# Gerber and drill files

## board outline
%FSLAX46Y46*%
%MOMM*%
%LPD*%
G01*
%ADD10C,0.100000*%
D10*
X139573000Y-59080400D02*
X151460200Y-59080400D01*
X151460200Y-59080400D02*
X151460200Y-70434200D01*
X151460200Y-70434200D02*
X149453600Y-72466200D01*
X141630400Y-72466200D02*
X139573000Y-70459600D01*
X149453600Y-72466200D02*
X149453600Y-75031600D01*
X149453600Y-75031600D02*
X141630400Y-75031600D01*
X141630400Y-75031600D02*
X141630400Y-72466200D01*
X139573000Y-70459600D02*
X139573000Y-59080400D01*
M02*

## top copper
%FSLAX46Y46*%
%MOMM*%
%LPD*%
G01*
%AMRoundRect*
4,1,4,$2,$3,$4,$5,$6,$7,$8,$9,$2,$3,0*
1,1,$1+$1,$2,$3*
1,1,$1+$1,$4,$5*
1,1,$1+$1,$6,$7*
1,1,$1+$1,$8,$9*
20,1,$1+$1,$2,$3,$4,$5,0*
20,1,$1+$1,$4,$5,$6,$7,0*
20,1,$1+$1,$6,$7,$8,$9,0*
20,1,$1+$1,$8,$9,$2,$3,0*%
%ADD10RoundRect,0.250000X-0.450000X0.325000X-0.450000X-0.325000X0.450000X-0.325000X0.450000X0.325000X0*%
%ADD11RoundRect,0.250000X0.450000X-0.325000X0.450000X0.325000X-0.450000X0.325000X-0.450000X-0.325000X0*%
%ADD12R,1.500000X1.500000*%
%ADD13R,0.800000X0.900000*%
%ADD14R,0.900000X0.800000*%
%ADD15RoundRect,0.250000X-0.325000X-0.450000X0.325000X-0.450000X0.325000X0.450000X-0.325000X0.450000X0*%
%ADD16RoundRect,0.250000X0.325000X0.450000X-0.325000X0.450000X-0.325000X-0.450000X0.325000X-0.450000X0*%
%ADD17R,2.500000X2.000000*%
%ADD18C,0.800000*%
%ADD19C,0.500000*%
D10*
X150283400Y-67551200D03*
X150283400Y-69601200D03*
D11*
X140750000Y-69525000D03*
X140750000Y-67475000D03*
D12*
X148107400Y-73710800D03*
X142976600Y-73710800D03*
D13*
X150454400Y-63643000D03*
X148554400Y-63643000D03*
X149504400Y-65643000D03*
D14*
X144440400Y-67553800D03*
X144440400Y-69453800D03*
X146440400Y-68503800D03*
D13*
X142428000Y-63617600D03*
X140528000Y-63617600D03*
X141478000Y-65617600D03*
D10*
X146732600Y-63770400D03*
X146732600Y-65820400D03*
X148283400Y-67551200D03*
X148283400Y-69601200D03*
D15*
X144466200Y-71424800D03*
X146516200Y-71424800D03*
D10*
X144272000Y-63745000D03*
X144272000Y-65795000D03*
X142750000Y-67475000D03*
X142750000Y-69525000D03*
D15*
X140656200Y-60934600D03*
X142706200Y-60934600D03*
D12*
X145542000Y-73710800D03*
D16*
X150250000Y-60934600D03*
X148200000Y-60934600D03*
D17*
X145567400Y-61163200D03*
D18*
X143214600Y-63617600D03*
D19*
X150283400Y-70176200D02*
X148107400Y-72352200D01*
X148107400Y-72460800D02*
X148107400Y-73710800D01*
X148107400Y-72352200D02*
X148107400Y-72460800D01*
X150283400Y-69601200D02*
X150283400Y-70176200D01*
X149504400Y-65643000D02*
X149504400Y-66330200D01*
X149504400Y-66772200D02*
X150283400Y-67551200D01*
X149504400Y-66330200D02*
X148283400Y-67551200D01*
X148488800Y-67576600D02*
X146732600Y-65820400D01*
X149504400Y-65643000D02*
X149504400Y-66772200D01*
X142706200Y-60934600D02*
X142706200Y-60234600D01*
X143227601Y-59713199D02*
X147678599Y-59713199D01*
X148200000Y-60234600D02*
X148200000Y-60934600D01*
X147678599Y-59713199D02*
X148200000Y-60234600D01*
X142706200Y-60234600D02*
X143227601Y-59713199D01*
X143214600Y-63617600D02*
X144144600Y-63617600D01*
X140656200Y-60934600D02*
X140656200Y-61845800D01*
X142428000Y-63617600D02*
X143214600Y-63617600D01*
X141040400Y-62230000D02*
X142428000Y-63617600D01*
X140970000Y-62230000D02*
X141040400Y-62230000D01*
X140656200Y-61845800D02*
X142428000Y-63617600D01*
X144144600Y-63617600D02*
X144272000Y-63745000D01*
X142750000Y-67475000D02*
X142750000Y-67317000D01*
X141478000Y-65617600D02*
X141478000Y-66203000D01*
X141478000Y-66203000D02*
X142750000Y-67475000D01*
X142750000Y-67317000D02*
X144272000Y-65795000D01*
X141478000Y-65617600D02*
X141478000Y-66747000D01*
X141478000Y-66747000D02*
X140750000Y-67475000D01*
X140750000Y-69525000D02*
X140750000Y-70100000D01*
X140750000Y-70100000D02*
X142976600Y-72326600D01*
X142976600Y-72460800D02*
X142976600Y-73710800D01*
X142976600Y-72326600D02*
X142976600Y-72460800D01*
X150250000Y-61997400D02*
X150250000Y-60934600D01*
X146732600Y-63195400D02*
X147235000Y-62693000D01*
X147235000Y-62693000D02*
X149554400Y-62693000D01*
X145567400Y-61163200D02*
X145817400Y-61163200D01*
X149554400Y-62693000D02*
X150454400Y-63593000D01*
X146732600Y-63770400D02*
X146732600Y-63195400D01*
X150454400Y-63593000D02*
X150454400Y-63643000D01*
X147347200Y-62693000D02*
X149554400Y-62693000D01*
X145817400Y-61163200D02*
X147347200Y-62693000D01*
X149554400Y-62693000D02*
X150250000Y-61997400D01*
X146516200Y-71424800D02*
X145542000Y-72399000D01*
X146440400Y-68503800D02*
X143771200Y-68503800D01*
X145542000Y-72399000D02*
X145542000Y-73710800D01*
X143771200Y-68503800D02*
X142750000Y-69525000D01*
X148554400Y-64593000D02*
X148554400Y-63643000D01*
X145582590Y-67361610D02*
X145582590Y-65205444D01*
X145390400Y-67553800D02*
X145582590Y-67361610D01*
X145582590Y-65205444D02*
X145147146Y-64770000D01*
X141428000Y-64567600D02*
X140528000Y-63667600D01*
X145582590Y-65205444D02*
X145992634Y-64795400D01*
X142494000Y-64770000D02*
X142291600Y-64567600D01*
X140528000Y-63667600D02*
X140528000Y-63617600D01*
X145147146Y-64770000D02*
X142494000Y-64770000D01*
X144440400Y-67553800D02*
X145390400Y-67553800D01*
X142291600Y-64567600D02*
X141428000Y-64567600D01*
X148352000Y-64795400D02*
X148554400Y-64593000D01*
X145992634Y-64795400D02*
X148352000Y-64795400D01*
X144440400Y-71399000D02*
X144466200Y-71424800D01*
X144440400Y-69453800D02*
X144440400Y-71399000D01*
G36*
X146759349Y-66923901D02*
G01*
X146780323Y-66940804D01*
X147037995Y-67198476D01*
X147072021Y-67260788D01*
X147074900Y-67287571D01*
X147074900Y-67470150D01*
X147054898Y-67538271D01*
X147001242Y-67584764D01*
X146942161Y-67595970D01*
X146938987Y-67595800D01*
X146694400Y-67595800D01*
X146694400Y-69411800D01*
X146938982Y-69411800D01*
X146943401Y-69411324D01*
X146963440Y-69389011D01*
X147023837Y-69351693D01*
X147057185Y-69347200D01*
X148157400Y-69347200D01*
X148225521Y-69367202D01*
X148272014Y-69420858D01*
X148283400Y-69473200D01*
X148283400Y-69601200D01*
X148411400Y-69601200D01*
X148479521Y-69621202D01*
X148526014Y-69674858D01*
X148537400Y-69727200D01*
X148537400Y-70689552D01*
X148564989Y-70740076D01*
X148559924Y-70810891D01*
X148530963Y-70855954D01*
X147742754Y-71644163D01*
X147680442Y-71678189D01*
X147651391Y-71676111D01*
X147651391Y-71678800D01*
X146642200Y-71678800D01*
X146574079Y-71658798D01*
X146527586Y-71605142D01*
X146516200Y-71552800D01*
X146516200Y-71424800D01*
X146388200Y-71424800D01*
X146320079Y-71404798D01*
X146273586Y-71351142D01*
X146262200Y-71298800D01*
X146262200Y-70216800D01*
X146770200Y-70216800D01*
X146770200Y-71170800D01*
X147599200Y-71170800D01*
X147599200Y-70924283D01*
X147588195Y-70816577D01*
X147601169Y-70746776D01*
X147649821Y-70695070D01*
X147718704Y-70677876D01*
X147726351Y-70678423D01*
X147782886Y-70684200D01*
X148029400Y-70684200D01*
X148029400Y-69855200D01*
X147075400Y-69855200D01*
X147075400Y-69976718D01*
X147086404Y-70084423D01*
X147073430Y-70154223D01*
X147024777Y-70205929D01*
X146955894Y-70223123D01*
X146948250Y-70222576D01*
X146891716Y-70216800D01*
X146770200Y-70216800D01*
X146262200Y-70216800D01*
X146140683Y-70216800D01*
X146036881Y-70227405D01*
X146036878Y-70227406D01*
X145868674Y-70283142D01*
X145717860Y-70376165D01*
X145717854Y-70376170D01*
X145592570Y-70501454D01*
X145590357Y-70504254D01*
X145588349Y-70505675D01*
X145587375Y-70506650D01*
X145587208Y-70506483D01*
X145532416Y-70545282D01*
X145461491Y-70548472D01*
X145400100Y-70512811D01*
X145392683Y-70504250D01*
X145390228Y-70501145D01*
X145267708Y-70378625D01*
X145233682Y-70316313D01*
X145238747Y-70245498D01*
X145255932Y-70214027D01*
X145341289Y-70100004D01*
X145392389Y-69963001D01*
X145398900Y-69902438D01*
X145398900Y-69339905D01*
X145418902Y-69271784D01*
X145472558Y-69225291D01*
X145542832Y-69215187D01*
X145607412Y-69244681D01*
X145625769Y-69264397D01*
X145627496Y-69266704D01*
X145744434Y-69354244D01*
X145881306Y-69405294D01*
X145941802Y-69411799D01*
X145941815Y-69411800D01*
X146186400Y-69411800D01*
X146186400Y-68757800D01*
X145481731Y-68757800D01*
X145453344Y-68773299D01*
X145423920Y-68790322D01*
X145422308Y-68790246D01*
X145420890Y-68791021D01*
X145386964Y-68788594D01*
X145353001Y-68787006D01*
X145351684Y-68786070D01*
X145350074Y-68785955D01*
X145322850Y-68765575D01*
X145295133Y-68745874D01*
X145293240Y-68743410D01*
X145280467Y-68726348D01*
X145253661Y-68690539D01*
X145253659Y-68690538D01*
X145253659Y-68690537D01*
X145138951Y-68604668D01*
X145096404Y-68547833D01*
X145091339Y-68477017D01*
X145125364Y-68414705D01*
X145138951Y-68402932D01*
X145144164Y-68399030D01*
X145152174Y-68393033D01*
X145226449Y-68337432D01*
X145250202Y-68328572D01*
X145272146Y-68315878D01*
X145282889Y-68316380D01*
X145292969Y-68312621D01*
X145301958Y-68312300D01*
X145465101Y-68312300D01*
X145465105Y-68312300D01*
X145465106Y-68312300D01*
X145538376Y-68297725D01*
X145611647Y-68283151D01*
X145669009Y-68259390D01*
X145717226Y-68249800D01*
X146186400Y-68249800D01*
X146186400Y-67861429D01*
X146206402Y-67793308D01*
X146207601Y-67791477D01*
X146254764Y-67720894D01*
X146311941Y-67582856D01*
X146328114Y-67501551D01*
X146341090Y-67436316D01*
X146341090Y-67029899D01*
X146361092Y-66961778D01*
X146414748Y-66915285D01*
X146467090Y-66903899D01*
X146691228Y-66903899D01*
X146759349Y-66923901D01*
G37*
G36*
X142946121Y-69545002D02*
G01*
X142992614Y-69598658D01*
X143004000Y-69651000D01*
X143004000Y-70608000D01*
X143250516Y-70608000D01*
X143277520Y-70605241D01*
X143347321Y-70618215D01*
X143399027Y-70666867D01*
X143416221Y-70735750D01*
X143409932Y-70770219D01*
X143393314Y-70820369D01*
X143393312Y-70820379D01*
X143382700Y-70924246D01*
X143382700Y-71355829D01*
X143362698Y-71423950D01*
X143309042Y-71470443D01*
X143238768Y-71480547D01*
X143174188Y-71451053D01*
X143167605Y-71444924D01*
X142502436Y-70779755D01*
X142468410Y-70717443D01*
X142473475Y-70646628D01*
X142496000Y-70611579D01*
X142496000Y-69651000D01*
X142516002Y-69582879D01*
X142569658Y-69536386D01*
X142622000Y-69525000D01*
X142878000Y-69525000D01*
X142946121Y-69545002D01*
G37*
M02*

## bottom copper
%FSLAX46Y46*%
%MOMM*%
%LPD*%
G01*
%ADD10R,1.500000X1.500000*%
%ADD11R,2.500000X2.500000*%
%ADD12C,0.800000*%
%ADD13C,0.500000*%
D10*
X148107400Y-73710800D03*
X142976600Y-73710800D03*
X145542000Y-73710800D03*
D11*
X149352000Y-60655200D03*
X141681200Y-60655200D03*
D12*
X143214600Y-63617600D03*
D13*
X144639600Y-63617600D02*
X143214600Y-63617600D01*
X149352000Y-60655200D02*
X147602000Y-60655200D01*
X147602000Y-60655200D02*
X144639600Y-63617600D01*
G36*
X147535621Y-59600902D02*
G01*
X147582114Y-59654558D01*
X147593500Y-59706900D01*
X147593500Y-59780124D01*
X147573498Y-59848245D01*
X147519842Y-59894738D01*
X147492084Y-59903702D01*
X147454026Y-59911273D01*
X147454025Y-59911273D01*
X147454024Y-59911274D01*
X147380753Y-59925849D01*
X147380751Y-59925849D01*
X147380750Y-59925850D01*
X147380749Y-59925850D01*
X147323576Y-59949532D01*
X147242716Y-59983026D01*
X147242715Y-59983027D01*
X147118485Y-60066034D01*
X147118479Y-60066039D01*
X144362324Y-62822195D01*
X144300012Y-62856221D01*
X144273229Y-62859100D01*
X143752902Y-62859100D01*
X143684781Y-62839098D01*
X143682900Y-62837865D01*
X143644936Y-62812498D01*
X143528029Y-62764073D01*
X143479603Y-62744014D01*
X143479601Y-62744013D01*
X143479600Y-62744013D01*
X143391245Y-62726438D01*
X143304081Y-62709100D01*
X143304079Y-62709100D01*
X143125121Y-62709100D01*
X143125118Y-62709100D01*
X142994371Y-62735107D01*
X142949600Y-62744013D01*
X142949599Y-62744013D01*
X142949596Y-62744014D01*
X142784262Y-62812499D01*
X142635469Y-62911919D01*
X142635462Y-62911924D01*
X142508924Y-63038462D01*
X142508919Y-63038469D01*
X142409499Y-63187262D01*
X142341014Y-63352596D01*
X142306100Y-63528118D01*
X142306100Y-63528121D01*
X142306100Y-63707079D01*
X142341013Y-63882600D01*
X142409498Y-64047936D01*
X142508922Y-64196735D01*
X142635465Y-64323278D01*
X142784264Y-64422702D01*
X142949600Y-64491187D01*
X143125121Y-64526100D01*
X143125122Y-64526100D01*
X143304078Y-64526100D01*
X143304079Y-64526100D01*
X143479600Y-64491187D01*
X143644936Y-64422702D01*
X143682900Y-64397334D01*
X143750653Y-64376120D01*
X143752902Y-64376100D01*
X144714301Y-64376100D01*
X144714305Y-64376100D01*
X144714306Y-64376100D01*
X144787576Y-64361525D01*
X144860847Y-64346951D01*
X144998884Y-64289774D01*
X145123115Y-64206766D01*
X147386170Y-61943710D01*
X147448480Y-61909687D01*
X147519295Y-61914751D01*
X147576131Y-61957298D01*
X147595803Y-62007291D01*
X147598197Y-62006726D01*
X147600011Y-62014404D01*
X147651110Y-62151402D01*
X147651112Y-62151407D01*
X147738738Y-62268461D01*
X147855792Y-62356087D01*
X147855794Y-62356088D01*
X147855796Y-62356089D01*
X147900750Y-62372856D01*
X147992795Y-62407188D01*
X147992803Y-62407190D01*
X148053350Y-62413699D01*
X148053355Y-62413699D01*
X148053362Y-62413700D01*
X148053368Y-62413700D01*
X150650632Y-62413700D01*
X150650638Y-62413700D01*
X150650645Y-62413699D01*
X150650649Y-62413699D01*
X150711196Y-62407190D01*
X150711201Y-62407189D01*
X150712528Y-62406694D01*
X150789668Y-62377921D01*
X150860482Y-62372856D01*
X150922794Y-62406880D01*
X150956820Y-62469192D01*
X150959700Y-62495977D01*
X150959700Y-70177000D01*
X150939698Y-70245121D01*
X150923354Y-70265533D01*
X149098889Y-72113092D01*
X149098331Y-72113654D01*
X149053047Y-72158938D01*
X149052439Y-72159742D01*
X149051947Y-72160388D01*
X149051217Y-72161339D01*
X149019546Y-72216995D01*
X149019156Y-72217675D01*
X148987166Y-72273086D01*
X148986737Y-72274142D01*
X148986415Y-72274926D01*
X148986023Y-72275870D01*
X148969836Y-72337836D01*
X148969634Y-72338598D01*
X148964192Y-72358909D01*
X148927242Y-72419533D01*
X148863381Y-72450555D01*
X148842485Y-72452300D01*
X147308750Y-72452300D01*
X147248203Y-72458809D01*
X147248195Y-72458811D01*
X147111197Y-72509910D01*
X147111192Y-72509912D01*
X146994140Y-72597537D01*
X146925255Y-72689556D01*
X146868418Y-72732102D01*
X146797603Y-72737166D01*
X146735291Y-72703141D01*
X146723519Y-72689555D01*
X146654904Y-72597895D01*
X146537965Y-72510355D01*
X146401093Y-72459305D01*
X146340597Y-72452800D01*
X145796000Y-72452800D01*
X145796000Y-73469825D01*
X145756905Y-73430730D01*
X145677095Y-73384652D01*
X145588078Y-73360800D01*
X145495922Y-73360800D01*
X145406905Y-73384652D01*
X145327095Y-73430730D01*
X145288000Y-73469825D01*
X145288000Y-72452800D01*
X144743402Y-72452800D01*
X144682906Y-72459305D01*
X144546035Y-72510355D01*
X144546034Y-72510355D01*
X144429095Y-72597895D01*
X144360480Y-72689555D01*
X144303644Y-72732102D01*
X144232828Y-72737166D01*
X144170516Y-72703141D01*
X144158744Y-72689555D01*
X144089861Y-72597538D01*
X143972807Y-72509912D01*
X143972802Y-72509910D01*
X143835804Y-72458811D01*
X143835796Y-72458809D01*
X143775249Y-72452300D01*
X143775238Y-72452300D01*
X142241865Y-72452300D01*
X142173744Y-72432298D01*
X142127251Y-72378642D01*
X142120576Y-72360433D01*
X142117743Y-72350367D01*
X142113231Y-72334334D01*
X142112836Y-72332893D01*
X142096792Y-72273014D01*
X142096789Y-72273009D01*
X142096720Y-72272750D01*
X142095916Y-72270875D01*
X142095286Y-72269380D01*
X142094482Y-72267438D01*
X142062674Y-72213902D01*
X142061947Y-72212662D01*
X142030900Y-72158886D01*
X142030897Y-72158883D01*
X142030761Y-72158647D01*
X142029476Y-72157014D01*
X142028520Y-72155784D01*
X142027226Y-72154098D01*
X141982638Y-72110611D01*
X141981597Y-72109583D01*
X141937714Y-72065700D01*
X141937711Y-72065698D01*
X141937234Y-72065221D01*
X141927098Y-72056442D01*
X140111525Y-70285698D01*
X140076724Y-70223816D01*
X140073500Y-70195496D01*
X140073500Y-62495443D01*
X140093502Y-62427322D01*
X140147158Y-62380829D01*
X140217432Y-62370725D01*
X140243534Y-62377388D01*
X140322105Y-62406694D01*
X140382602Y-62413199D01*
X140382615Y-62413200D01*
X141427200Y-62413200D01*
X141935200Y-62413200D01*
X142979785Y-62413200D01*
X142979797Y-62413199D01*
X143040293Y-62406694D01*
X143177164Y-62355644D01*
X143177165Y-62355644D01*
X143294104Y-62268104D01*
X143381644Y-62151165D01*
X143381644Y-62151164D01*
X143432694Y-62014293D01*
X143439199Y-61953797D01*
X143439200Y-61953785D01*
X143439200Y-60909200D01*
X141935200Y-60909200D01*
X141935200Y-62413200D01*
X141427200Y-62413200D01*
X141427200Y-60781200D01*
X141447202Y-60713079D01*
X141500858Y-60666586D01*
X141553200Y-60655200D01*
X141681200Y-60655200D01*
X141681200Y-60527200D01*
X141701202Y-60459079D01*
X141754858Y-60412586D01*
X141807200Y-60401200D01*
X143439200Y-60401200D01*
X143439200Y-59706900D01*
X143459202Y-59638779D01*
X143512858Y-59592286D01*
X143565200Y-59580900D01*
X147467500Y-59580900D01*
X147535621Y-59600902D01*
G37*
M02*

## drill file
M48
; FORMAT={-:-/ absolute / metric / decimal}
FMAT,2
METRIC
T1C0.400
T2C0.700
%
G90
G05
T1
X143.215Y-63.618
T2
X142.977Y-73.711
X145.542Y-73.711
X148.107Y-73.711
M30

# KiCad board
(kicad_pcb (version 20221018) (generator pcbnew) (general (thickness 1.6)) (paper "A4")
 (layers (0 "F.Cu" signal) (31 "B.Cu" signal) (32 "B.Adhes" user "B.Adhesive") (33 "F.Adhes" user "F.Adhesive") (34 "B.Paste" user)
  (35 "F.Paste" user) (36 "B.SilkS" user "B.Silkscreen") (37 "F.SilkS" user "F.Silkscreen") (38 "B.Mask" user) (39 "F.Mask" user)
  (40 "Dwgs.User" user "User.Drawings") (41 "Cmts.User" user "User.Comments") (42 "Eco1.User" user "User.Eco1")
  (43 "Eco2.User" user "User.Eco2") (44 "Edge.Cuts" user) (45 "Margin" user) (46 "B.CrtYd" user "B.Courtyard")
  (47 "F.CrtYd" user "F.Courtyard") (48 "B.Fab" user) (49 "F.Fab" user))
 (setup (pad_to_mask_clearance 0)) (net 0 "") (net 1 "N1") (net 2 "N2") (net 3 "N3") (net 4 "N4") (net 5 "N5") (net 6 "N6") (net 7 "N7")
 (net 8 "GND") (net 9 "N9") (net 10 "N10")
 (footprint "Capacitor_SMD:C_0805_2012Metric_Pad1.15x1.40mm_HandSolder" (layer "F.Cu") (at 150.2834 68.5762 -90)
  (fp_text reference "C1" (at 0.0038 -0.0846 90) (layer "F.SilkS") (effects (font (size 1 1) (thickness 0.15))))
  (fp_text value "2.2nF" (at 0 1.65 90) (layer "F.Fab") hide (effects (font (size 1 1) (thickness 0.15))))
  (pad "1" smd roundrect (at -1.025 0 270) (size 1.15 1.4) (layers "F.Cu" "F.Paste" "F.Mask") (roundrect_rratio 0.217391) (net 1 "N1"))
  (pad "2" smd roundrect (at 1.025 0 270) (size 1.15 1.4) (layers "F.Cu" "F.Paste" "F.Mask") (roundrect_rratio 0.217391) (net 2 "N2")))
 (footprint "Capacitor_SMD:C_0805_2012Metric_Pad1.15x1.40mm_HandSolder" (layer "F.Cu") (at 140.75 68.5 90)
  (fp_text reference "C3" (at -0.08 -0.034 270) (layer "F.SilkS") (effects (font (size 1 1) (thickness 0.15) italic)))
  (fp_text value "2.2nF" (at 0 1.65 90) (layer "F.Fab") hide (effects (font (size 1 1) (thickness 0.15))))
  (pad "1" smd roundrect (at -1.025 0 90) (size 1.15 1.4) (layers "F.Cu" "F.Paste" "F.Mask") (roundrect_rratio 0.217391) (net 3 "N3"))
  (pad "2" smd roundrect (at 1.025 0 90) (size 1.15 1.4) (layers "F.Cu" "F.Paste" "F.Mask") (roundrect_rratio 0.217391) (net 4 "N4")))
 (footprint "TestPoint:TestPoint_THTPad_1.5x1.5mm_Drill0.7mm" (layer "F.Cu") (at 148.1074 73.7108)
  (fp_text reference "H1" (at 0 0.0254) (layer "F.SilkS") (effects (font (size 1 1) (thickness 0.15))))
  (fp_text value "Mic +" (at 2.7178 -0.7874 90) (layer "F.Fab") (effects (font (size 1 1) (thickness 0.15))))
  (pad "M-" thru_hole rect (at 0 0) (size 1.5 1.5) (drill 0.7) (layers "*.Cu" "*.Mask") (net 2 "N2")))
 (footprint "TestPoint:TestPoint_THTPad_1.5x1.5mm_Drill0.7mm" (layer "F.Cu") (at 142.9766 73.7108)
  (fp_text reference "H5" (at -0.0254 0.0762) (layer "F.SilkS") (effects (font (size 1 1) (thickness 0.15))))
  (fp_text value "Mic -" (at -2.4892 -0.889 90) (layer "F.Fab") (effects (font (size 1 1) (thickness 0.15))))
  (pad "M+" thru_hole rect (at 0 0) (size 1.5 1.5) (drill 0.7) (layers "*.Cu" "*.Mask") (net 3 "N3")))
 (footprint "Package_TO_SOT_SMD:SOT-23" (layer "F.Cu") (at 149.5044 64.643 -90)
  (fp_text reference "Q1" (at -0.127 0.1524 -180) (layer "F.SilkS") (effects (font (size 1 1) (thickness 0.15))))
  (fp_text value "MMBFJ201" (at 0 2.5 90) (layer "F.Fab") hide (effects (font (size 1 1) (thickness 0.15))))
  (pad "1" smd rect (at -1 -0.95 270) (size 0.9 0.8) (layers "F.Cu" "F.Paste" "F.Mask") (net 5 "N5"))
  (pad "2" smd rect (at -1 0.95 270) (size 0.9 0.8) (layers "F.Cu" "F.Paste" "F.Mask") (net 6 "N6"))
  (pad "3" smd rect (at 1 0 270) (size 0.9 0.8) (layers "F.Cu" "F.Paste" "F.Mask") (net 1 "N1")))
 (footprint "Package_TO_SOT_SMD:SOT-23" (layer "F.Cu") (at 145.4404 68.5038)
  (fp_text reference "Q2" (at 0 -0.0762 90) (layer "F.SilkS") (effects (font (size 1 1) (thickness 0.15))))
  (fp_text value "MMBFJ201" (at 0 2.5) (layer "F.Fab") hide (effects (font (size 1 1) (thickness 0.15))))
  (pad "1" smd rect (at -1 -0.95) (size 0.9 0.8) (layers "F.Cu" "F.Paste" "F.Mask") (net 6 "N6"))
  (pad "2" smd rect (at -1 0.95) (size 0.9 0.8) (layers "F.Cu" "F.Paste" "F.Mask") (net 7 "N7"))
  (pad "3" smd rect (at 1 0) (size 0.9 0.8) (layers "F.Cu" "F.Paste" "F.Mask") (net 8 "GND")))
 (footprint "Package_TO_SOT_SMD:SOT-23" (layer "F.Cu") (at 141.478 64.6176 -90)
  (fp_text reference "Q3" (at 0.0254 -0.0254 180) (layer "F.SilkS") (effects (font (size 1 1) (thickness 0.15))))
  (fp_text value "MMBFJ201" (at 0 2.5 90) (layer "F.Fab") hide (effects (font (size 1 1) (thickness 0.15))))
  (pad "1" smd rect (at -1 -0.95 270) (size 0.9 0.8) (layers "F.Cu" "F.Paste" "F.Mask") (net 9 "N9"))
  (pad "2" smd rect (at -1 0.95 270) (size 0.9 0.8) (layers "F.Cu" "F.Paste" "F.Mask") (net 6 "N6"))
  (pad "3" smd rect (at 1 0 270) (size 0.9 0.8) (layers "F.Cu" "F.Paste" "F.Mask") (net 4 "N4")))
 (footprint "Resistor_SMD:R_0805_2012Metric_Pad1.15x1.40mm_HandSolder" (layer "F.Cu") (at 146.7326 64.7954 -90)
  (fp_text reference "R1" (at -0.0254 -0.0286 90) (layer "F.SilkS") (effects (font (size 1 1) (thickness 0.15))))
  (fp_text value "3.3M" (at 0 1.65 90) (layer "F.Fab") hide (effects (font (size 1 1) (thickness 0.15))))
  (pad "1" smd roundrect (at -1.025 0 270) (size 1.15 1.4) (layers "F.Cu" "F.Paste" "F.Mask") (roundrect_rratio 0.217391) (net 5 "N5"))
  (pad "2" smd roundrect (at 1.025 0 270) (size 1.15 1.4) (layers "F.Cu" "F.Paste" "F.Mask") (roundrect_rratio 0.217391) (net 1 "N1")))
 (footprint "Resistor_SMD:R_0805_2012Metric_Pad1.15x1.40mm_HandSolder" (layer "F.Cu") (at 148.2834 68.5762 -90)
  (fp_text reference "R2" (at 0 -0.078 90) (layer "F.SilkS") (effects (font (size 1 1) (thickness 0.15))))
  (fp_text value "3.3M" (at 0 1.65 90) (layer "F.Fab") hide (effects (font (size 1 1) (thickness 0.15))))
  (pad "1" smd roundrect (at -1.025 0 270) (size 1.15 1.4) (layers "F.Cu" "F.Paste" "F.Mask") (roundrect_rratio 0.217391) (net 1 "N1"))
  (pad "2" smd roundrect (at 1.025 0 270) (size 1.15 1.4) (layers "F.Cu" "F.Paste" "F.Mask") (roundrect_rratio 0.217391) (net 8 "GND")))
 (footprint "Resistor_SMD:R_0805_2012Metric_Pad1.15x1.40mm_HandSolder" (layer "F.Cu") (at 145.4912 71.4248)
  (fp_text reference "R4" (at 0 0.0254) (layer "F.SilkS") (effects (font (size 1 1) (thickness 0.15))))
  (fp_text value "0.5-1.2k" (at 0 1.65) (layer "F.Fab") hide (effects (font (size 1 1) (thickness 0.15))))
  (pad "1" smd roundrect (at -1.025 0) (size 1.15 1.4) (layers "F.Cu" "F.Paste" "F.Mask") (roundrect_rratio 0.217391) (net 7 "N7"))
  (pad "2" smd roundrect (at 1.025 0) (size 1.15 1.4) (layers "F.Cu" "F.Paste" "F.Mask") (roundrect_rratio 0.217391) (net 8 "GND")))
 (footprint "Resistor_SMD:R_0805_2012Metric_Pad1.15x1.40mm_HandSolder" (layer "F.Cu") (at 144.272 64.77 -90)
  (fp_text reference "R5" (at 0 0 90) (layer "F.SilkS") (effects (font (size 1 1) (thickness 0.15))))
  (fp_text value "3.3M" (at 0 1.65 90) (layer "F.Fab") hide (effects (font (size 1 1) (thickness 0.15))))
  (pad "1" smd roundrect (at -1.025 0 270) (size 1.15 1.4) (layers "F.Cu" "F.Paste" "F.Mask") (roundrect_rratio 0.217391) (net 9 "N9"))
  (pad "2" smd roundrect (at 1.025 0 270) (size 1.15 1.4) (layers "F.Cu" "F.Paste" "F.Mask") (roundrect_rratio 0.217391) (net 4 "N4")))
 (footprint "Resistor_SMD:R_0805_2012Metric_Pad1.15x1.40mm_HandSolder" (layer "F.Cu") (at 142.75 68.5 -90)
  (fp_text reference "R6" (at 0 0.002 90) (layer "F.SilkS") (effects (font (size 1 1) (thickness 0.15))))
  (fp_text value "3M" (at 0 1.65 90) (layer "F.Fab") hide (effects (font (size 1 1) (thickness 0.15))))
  (pad "1" smd roundrect (at -1.025 0 270) (size 1.15 1.4) (layers "F.Cu" "F.Paste" "F.Mask") (roundrect_rratio 0.217391) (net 4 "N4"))
  (pad "2" smd roundrect (at 1.025 0 270) (size 1.15 1.4) (layers "F.Cu" "F.Paste" "F.Mask") (roundrect_rratio 0.217391) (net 8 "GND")))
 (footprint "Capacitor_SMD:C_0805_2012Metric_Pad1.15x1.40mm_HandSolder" (layer "F.Cu") (at 141.6812 60.9346)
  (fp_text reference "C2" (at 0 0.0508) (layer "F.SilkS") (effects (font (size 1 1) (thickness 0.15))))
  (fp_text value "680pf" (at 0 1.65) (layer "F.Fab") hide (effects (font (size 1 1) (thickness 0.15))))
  (pad "1" smd roundrect (at -1.025 0) (size 1.15 1.4) (layers "F.Cu" "F.Paste" "F.Mask") (roundrect_rratio 0.217391) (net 9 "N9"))
  (pad "2" smd roundrect (at 1.025 0) (size 1.15 1.4) (layers "F.Cu" "F.Paste" "F.Mask") (roundrect_rratio 0.217391) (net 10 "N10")))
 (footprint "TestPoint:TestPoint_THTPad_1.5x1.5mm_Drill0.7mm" (layer "F.Cu") (at 145.542 73.7108)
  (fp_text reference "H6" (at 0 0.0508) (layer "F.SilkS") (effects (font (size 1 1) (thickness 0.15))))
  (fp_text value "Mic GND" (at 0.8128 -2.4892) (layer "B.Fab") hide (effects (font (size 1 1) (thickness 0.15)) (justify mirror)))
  (pad "GND" thru_hole rect (at 0 0) (size 1.5 1.5) (drill 0.7) (layers "*.Cu" "*.Mask") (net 8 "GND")))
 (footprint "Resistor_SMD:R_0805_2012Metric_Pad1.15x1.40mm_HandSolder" (layer "F.Cu") (at 149.225 60.9346 180)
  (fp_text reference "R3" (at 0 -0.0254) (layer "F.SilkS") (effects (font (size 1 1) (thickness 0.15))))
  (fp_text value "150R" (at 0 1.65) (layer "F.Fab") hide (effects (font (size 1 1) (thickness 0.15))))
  (pad "1" smd roundrect (at -1.025 0 180) (size 1.15 1.4) (layers "F.Cu" "F.Paste" "F.Mask") (roundrect_rratio 0.217391) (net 5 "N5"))
  (pad "2" smd roundrect (at 1.025 0 180) (size 1.15 1.4) (layers "F.Cu" "F.Paste" "F.Mask") (roundrect_rratio 0.217391) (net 10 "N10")))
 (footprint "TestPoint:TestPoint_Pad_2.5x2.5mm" (layer "F.Cu") (at 145.5674 61.1632)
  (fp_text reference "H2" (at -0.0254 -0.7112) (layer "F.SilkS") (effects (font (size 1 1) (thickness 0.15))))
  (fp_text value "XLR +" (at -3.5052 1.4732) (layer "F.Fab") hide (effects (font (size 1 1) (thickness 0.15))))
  (pad "-" smd rect (at 0 0) (size 2.5 2) (layers "F.Cu" "F.Mask") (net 5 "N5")))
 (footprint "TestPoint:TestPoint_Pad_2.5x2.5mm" (layer "B.Cu") (at 149.352 60.6552)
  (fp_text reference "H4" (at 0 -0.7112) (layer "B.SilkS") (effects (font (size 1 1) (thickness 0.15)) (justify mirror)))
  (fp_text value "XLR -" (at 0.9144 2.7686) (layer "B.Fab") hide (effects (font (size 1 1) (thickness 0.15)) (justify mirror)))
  (pad "+" smd rect (at 0 0) (size 2.5 2.5) (layers "B.Cu" "B.Mask") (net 9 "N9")))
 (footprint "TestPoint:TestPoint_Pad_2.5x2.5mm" (layer "B.Cu") (at 141.6812 60.6552)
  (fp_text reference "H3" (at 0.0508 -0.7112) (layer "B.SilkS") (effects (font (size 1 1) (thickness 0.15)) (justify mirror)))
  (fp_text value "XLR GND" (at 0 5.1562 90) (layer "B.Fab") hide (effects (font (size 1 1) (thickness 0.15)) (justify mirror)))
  (pad "GND" smd rect (at 0 0) (size 2.5 2.5) (layers "B.Cu" "B.Mask") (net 8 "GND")))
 (gr_line (start 139.573 59.0804) (end 151.4602 59.0804) (stroke (width 0.1) (type solid)) (layer "Edge.Cuts"))
 (gr_line (start 151.4602 59.0804) (end 151.4602 70.4342) (stroke (width 0.1) (type solid)) (layer "Edge.Cuts"))
 (gr_line (start 151.4602 70.4342) (end 149.4536 72.4662) (stroke (width 0.1) (type solid)) (layer "Edge.Cuts"))
 (gr_line (start 141.6304 72.4662) (end 139.573 70.4596) (stroke (width 0.1) (type solid)) (layer "Edge.Cuts"))
 (gr_line (start 149.4536 72.4662) (end 149.4536 75.0316) (stroke (width 0.1) (type solid)) (layer "Edge.Cuts"))
 (gr_line (start 149.4536 75.0316) (end 141.6304 75.0316) (stroke (width 0.1) (type solid)) (layer "Edge.Cuts"))
 (gr_line (start 141.6304 75.0316) (end 141.6304 72.4662) (stroke (width 0.1) (type solid)) (layer "Edge.Cuts"))
 (gr_line (start 139.573 70.4596) (end 139.573 59.0804) (stroke (width 0.1) (type solid)) (layer "Edge.Cuts"))
 (segment (start 150.2834 70.1762) (end 148.1074 72.3522) (width 0.5) (layer "F.Cu") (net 2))
 (segment (start 148.1074 72.4608) (end 148.1074 73.7108) (width 0.5) (layer "F.Cu") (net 2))
 (segment (start 148.1074 72.3522) (end 148.1074 72.4608) (width 0.5) (layer "F.Cu") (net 2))
 (segment (start 150.2834 69.6012) (end 150.2834 70.1762) (width 0.5) (layer "F.Cu") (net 2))
 (segment (start 149.5044 65.643) (end 149.5044 66.3302) (width 0.5) (layer "F.Cu") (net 1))
 (segment (start 149.5044 66.7722) (end 150.2834 67.5512) (width 0.5) (layer "F.Cu") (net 1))
 (segment (start 149.5044 66.3302) (end 148.2834 67.5512) (width 0.5) (layer "F.Cu") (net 1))
 (segment (start 148.4888 67.5766) (end 146.7326 65.8204) (width 0.5) (layer "F.Cu") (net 1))
 (segment (start 149.5044 65.643) (end 149.5044 66.7722) (width 0.5) (layer "F.Cu") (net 1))
 (segment (start 142.7062 60.9346) (end 142.7062 60.2346) (width 0.5) (layer "F.Cu") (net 10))
 (segment (start 143.227601 59.713199) (end 147.678599 59.713199) (width 0.5) (layer "F.Cu") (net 10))
 (segment (start 148.2 60.2346) (end 148.2 60.9346) (width 0.5) (layer "F.Cu") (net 10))
 (segment (start 147.678599 59.713199) (end 148.2 60.2346) (width 0.5) (layer "F.Cu") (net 10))
 (segment (start 142.7062 60.2346) (end 143.227601 59.713199) (width 0.5) (layer "F.Cu") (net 10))
 (segment (start 143.2146 63.6176) (end 144.1446 63.6176) (width 0.5) (layer "F.Cu") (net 9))
 (segment (start 140.6562 60.9346) (end 140.6562 61.8458) (width 0.5) (layer "F.Cu") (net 9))
 (segment (start 142.428 63.6176) (end 143.2146 63.6176) (width 0.5) (layer "F.Cu") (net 9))
 (segment (start 141.0404 62.23) (end 142.428 63.6176) (width 0.5) (layer "F.Cu") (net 9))
 (segment (start 140.97 62.23) (end 141.0404 62.23) (width 0.5) (layer "F.Cu") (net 9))
 (segment (start 140.6562 61.8458) (end 142.428 63.6176) (width 0.5) (layer "F.Cu") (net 9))
 (segment (start 144.1446 63.6176) (end 144.272 63.745) (width 0.5) (layer "F.Cu") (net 9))
 (via (at 143.2146 63.6176) (size 0.8) (drill 0.4) (layers "F.Cu" "B.Cu") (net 9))
 (segment (start 144.6396 63.6176) (end 143.2146 63.6176) (width 0.5) (layer "B.Cu") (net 9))
 (segment (start 149.352 60.6552) (end 147.602 60.6552) (width 0.5) (layer "B.Cu") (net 9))
 (segment (start 147.602 60.6552) (end 144.6396 63.6176) (width 0.5) (layer "B.Cu") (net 9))
 (segment (start 142.75 67.475) (end 142.75 67.317) (width 0.5) (layer "F.Cu") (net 4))
 (segment (start 141.478 65.6176) (end 141.478 66.203) (width 0.5) (layer "F.Cu") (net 4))
 (segment (start 141.478 66.203) (end 142.75 67.475) (width 0.5) (layer "F.Cu") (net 4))
 (segment (start 142.75 67.317) (end 144.272 65.795) (width 0.5) (layer "F.Cu") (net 4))
 (segment (start 141.478 65.6176) (end 141.478 66.747) (width 0.5) (layer "F.Cu") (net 4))
 (segment (start 141.478 66.747) (end 140.75 67.475) (width 0.5) (layer "F.Cu") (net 4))
 (segment (start 140.75 69.525) (end 140.75 70.1) (width 0.5) (layer "F.Cu") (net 3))
 (segment (start 140.75 70.1) (end 142.9766 72.3266) (width 0.5) (layer "F.Cu") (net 3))
 (segment (start 142.9766 72.4608) (end 142.9766 73.7108) (width 0.5) (layer "F.Cu") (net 3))
 (segment (start 142.9766 72.3266) (end 142.9766 72.4608) (width 0.5) (layer "F.Cu") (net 3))
 (segment (start 150.25 61.9974) (end 150.25 60.9346) (width 0.5) (layer "F.Cu") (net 5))
 (segment (start 146.7326 63.1954) (end 147.235 62.693) (width 0.5) (layer "F.Cu") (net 5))
 (segment (start 147.235 62.693) (end 149.5544 62.693) (width 0.5) (layer "F.Cu") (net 5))
 (segment (start 145.5674 61.1632) (end 145.8174 61.1632) (width 0.5) (layer "F.Cu") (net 5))
 (segment (start 149.5544 62.693) (end 150.4544 63.593) (width 0.5) (layer "F.Cu") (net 5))
 (segment (start 146.7326 63.7704) (end 146.7326 63.1954) (width 0.5) (layer "F.Cu") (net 5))
 (segment (start 150.4544 63.593) (end 150.4544 63.643) (width 0.5) (layer "F.Cu") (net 5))
 (segment (start 147.3472 62.693) (end 149.5544 62.693) (width 0.5) (layer "F.Cu") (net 5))
 (segment (start 145.8174 61.1632) (end 147.3472 62.693) (width 0.5) (layer "F.Cu") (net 5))
 (segment (start 149.5544 62.693) (end 150.25 61.9974) (width 0.5) (layer "F.Cu") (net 5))
 (segment (start 146.5162 71.4248) (end 145.542 72.399) (width 0.5) (layer "F.Cu") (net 8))
 (segment (start 146.4404 68.5038) (end 143.7712 68.5038) (width 0.5) (layer "F.Cu") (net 8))
 (segment (start 145.542 72.399) (end 145.542 73.7108) (width 0.5) (layer "F.Cu") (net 8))
 (segment (start 143.7712 68.5038) (end 142.75 69.525) (width 0.5) (layer "F.Cu") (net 8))
 (segment (start 148.5544 64.593) (end 148.5544 63.643) (width 0.5) (layer "F.Cu") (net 6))
 (segment (start 145.58259 67.36161) (end 145.58259 65.205444) (width 0.5) (layer "F.Cu") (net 6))
 (segment (start 145.3904 67.5538) (end 145.58259 67.36161) (width 0.5) (layer "F.Cu") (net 6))
 (segment (start 145.58259 65.205444) (end 145.147146 64.77) (width 0.5) (layer "F.Cu") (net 6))
 (segment (start 141.428 64.5676) (end 140.528 63.6676) (width 0.5) (layer "F.Cu") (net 6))
 (segment (start 145.58259 65.205444) (end 145.992634 64.7954) (width 0.5) (layer "F.Cu") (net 6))
 (segment (start 142.494 64.77) (end 142.2916 64.5676) (width 0.5) (layer "F.Cu") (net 6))
 (segment (start 140.528 63.6676) (end 140.528 63.6176) (width 0.5) (layer "F.Cu") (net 6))
 (segment (start 145.147146 64.77) (end 142.494 64.77) (width 0.5) (layer "F.Cu") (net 6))
 (segment (start 144.4404 67.5538) (end 145.3904 67.5538) (width 0.5) (layer "F.Cu") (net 6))
 (segment (start 142.2916 64.5676) (end 141.428 64.5676) (width 0.5) (layer "F.Cu") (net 6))
 (segment (start 148.352 64.7954) (end 148.5544 64.593) (width 0.5) (layer "F.Cu") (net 6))
 (segment (start 145.992634 64.7954) (end 148.352 64.7954) (width 0.5) (layer "F.Cu") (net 6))
 (segment (start 144.4404 71.399) (end 144.4662 71.4248) (width 0.5) (layer "F.Cu") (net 7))
 (segment (start 144.4404 69.4538) (end 144.4404 71.399) (width 0.5) (layer "F.Cu") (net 7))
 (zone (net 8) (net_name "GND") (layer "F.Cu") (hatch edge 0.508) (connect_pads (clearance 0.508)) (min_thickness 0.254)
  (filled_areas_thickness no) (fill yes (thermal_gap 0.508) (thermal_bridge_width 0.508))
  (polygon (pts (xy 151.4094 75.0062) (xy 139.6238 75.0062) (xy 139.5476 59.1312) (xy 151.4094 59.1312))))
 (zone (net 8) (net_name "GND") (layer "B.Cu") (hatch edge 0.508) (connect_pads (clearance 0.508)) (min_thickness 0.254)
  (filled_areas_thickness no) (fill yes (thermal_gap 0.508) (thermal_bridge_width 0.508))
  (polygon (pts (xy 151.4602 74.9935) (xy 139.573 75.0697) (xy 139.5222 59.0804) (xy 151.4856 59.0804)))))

